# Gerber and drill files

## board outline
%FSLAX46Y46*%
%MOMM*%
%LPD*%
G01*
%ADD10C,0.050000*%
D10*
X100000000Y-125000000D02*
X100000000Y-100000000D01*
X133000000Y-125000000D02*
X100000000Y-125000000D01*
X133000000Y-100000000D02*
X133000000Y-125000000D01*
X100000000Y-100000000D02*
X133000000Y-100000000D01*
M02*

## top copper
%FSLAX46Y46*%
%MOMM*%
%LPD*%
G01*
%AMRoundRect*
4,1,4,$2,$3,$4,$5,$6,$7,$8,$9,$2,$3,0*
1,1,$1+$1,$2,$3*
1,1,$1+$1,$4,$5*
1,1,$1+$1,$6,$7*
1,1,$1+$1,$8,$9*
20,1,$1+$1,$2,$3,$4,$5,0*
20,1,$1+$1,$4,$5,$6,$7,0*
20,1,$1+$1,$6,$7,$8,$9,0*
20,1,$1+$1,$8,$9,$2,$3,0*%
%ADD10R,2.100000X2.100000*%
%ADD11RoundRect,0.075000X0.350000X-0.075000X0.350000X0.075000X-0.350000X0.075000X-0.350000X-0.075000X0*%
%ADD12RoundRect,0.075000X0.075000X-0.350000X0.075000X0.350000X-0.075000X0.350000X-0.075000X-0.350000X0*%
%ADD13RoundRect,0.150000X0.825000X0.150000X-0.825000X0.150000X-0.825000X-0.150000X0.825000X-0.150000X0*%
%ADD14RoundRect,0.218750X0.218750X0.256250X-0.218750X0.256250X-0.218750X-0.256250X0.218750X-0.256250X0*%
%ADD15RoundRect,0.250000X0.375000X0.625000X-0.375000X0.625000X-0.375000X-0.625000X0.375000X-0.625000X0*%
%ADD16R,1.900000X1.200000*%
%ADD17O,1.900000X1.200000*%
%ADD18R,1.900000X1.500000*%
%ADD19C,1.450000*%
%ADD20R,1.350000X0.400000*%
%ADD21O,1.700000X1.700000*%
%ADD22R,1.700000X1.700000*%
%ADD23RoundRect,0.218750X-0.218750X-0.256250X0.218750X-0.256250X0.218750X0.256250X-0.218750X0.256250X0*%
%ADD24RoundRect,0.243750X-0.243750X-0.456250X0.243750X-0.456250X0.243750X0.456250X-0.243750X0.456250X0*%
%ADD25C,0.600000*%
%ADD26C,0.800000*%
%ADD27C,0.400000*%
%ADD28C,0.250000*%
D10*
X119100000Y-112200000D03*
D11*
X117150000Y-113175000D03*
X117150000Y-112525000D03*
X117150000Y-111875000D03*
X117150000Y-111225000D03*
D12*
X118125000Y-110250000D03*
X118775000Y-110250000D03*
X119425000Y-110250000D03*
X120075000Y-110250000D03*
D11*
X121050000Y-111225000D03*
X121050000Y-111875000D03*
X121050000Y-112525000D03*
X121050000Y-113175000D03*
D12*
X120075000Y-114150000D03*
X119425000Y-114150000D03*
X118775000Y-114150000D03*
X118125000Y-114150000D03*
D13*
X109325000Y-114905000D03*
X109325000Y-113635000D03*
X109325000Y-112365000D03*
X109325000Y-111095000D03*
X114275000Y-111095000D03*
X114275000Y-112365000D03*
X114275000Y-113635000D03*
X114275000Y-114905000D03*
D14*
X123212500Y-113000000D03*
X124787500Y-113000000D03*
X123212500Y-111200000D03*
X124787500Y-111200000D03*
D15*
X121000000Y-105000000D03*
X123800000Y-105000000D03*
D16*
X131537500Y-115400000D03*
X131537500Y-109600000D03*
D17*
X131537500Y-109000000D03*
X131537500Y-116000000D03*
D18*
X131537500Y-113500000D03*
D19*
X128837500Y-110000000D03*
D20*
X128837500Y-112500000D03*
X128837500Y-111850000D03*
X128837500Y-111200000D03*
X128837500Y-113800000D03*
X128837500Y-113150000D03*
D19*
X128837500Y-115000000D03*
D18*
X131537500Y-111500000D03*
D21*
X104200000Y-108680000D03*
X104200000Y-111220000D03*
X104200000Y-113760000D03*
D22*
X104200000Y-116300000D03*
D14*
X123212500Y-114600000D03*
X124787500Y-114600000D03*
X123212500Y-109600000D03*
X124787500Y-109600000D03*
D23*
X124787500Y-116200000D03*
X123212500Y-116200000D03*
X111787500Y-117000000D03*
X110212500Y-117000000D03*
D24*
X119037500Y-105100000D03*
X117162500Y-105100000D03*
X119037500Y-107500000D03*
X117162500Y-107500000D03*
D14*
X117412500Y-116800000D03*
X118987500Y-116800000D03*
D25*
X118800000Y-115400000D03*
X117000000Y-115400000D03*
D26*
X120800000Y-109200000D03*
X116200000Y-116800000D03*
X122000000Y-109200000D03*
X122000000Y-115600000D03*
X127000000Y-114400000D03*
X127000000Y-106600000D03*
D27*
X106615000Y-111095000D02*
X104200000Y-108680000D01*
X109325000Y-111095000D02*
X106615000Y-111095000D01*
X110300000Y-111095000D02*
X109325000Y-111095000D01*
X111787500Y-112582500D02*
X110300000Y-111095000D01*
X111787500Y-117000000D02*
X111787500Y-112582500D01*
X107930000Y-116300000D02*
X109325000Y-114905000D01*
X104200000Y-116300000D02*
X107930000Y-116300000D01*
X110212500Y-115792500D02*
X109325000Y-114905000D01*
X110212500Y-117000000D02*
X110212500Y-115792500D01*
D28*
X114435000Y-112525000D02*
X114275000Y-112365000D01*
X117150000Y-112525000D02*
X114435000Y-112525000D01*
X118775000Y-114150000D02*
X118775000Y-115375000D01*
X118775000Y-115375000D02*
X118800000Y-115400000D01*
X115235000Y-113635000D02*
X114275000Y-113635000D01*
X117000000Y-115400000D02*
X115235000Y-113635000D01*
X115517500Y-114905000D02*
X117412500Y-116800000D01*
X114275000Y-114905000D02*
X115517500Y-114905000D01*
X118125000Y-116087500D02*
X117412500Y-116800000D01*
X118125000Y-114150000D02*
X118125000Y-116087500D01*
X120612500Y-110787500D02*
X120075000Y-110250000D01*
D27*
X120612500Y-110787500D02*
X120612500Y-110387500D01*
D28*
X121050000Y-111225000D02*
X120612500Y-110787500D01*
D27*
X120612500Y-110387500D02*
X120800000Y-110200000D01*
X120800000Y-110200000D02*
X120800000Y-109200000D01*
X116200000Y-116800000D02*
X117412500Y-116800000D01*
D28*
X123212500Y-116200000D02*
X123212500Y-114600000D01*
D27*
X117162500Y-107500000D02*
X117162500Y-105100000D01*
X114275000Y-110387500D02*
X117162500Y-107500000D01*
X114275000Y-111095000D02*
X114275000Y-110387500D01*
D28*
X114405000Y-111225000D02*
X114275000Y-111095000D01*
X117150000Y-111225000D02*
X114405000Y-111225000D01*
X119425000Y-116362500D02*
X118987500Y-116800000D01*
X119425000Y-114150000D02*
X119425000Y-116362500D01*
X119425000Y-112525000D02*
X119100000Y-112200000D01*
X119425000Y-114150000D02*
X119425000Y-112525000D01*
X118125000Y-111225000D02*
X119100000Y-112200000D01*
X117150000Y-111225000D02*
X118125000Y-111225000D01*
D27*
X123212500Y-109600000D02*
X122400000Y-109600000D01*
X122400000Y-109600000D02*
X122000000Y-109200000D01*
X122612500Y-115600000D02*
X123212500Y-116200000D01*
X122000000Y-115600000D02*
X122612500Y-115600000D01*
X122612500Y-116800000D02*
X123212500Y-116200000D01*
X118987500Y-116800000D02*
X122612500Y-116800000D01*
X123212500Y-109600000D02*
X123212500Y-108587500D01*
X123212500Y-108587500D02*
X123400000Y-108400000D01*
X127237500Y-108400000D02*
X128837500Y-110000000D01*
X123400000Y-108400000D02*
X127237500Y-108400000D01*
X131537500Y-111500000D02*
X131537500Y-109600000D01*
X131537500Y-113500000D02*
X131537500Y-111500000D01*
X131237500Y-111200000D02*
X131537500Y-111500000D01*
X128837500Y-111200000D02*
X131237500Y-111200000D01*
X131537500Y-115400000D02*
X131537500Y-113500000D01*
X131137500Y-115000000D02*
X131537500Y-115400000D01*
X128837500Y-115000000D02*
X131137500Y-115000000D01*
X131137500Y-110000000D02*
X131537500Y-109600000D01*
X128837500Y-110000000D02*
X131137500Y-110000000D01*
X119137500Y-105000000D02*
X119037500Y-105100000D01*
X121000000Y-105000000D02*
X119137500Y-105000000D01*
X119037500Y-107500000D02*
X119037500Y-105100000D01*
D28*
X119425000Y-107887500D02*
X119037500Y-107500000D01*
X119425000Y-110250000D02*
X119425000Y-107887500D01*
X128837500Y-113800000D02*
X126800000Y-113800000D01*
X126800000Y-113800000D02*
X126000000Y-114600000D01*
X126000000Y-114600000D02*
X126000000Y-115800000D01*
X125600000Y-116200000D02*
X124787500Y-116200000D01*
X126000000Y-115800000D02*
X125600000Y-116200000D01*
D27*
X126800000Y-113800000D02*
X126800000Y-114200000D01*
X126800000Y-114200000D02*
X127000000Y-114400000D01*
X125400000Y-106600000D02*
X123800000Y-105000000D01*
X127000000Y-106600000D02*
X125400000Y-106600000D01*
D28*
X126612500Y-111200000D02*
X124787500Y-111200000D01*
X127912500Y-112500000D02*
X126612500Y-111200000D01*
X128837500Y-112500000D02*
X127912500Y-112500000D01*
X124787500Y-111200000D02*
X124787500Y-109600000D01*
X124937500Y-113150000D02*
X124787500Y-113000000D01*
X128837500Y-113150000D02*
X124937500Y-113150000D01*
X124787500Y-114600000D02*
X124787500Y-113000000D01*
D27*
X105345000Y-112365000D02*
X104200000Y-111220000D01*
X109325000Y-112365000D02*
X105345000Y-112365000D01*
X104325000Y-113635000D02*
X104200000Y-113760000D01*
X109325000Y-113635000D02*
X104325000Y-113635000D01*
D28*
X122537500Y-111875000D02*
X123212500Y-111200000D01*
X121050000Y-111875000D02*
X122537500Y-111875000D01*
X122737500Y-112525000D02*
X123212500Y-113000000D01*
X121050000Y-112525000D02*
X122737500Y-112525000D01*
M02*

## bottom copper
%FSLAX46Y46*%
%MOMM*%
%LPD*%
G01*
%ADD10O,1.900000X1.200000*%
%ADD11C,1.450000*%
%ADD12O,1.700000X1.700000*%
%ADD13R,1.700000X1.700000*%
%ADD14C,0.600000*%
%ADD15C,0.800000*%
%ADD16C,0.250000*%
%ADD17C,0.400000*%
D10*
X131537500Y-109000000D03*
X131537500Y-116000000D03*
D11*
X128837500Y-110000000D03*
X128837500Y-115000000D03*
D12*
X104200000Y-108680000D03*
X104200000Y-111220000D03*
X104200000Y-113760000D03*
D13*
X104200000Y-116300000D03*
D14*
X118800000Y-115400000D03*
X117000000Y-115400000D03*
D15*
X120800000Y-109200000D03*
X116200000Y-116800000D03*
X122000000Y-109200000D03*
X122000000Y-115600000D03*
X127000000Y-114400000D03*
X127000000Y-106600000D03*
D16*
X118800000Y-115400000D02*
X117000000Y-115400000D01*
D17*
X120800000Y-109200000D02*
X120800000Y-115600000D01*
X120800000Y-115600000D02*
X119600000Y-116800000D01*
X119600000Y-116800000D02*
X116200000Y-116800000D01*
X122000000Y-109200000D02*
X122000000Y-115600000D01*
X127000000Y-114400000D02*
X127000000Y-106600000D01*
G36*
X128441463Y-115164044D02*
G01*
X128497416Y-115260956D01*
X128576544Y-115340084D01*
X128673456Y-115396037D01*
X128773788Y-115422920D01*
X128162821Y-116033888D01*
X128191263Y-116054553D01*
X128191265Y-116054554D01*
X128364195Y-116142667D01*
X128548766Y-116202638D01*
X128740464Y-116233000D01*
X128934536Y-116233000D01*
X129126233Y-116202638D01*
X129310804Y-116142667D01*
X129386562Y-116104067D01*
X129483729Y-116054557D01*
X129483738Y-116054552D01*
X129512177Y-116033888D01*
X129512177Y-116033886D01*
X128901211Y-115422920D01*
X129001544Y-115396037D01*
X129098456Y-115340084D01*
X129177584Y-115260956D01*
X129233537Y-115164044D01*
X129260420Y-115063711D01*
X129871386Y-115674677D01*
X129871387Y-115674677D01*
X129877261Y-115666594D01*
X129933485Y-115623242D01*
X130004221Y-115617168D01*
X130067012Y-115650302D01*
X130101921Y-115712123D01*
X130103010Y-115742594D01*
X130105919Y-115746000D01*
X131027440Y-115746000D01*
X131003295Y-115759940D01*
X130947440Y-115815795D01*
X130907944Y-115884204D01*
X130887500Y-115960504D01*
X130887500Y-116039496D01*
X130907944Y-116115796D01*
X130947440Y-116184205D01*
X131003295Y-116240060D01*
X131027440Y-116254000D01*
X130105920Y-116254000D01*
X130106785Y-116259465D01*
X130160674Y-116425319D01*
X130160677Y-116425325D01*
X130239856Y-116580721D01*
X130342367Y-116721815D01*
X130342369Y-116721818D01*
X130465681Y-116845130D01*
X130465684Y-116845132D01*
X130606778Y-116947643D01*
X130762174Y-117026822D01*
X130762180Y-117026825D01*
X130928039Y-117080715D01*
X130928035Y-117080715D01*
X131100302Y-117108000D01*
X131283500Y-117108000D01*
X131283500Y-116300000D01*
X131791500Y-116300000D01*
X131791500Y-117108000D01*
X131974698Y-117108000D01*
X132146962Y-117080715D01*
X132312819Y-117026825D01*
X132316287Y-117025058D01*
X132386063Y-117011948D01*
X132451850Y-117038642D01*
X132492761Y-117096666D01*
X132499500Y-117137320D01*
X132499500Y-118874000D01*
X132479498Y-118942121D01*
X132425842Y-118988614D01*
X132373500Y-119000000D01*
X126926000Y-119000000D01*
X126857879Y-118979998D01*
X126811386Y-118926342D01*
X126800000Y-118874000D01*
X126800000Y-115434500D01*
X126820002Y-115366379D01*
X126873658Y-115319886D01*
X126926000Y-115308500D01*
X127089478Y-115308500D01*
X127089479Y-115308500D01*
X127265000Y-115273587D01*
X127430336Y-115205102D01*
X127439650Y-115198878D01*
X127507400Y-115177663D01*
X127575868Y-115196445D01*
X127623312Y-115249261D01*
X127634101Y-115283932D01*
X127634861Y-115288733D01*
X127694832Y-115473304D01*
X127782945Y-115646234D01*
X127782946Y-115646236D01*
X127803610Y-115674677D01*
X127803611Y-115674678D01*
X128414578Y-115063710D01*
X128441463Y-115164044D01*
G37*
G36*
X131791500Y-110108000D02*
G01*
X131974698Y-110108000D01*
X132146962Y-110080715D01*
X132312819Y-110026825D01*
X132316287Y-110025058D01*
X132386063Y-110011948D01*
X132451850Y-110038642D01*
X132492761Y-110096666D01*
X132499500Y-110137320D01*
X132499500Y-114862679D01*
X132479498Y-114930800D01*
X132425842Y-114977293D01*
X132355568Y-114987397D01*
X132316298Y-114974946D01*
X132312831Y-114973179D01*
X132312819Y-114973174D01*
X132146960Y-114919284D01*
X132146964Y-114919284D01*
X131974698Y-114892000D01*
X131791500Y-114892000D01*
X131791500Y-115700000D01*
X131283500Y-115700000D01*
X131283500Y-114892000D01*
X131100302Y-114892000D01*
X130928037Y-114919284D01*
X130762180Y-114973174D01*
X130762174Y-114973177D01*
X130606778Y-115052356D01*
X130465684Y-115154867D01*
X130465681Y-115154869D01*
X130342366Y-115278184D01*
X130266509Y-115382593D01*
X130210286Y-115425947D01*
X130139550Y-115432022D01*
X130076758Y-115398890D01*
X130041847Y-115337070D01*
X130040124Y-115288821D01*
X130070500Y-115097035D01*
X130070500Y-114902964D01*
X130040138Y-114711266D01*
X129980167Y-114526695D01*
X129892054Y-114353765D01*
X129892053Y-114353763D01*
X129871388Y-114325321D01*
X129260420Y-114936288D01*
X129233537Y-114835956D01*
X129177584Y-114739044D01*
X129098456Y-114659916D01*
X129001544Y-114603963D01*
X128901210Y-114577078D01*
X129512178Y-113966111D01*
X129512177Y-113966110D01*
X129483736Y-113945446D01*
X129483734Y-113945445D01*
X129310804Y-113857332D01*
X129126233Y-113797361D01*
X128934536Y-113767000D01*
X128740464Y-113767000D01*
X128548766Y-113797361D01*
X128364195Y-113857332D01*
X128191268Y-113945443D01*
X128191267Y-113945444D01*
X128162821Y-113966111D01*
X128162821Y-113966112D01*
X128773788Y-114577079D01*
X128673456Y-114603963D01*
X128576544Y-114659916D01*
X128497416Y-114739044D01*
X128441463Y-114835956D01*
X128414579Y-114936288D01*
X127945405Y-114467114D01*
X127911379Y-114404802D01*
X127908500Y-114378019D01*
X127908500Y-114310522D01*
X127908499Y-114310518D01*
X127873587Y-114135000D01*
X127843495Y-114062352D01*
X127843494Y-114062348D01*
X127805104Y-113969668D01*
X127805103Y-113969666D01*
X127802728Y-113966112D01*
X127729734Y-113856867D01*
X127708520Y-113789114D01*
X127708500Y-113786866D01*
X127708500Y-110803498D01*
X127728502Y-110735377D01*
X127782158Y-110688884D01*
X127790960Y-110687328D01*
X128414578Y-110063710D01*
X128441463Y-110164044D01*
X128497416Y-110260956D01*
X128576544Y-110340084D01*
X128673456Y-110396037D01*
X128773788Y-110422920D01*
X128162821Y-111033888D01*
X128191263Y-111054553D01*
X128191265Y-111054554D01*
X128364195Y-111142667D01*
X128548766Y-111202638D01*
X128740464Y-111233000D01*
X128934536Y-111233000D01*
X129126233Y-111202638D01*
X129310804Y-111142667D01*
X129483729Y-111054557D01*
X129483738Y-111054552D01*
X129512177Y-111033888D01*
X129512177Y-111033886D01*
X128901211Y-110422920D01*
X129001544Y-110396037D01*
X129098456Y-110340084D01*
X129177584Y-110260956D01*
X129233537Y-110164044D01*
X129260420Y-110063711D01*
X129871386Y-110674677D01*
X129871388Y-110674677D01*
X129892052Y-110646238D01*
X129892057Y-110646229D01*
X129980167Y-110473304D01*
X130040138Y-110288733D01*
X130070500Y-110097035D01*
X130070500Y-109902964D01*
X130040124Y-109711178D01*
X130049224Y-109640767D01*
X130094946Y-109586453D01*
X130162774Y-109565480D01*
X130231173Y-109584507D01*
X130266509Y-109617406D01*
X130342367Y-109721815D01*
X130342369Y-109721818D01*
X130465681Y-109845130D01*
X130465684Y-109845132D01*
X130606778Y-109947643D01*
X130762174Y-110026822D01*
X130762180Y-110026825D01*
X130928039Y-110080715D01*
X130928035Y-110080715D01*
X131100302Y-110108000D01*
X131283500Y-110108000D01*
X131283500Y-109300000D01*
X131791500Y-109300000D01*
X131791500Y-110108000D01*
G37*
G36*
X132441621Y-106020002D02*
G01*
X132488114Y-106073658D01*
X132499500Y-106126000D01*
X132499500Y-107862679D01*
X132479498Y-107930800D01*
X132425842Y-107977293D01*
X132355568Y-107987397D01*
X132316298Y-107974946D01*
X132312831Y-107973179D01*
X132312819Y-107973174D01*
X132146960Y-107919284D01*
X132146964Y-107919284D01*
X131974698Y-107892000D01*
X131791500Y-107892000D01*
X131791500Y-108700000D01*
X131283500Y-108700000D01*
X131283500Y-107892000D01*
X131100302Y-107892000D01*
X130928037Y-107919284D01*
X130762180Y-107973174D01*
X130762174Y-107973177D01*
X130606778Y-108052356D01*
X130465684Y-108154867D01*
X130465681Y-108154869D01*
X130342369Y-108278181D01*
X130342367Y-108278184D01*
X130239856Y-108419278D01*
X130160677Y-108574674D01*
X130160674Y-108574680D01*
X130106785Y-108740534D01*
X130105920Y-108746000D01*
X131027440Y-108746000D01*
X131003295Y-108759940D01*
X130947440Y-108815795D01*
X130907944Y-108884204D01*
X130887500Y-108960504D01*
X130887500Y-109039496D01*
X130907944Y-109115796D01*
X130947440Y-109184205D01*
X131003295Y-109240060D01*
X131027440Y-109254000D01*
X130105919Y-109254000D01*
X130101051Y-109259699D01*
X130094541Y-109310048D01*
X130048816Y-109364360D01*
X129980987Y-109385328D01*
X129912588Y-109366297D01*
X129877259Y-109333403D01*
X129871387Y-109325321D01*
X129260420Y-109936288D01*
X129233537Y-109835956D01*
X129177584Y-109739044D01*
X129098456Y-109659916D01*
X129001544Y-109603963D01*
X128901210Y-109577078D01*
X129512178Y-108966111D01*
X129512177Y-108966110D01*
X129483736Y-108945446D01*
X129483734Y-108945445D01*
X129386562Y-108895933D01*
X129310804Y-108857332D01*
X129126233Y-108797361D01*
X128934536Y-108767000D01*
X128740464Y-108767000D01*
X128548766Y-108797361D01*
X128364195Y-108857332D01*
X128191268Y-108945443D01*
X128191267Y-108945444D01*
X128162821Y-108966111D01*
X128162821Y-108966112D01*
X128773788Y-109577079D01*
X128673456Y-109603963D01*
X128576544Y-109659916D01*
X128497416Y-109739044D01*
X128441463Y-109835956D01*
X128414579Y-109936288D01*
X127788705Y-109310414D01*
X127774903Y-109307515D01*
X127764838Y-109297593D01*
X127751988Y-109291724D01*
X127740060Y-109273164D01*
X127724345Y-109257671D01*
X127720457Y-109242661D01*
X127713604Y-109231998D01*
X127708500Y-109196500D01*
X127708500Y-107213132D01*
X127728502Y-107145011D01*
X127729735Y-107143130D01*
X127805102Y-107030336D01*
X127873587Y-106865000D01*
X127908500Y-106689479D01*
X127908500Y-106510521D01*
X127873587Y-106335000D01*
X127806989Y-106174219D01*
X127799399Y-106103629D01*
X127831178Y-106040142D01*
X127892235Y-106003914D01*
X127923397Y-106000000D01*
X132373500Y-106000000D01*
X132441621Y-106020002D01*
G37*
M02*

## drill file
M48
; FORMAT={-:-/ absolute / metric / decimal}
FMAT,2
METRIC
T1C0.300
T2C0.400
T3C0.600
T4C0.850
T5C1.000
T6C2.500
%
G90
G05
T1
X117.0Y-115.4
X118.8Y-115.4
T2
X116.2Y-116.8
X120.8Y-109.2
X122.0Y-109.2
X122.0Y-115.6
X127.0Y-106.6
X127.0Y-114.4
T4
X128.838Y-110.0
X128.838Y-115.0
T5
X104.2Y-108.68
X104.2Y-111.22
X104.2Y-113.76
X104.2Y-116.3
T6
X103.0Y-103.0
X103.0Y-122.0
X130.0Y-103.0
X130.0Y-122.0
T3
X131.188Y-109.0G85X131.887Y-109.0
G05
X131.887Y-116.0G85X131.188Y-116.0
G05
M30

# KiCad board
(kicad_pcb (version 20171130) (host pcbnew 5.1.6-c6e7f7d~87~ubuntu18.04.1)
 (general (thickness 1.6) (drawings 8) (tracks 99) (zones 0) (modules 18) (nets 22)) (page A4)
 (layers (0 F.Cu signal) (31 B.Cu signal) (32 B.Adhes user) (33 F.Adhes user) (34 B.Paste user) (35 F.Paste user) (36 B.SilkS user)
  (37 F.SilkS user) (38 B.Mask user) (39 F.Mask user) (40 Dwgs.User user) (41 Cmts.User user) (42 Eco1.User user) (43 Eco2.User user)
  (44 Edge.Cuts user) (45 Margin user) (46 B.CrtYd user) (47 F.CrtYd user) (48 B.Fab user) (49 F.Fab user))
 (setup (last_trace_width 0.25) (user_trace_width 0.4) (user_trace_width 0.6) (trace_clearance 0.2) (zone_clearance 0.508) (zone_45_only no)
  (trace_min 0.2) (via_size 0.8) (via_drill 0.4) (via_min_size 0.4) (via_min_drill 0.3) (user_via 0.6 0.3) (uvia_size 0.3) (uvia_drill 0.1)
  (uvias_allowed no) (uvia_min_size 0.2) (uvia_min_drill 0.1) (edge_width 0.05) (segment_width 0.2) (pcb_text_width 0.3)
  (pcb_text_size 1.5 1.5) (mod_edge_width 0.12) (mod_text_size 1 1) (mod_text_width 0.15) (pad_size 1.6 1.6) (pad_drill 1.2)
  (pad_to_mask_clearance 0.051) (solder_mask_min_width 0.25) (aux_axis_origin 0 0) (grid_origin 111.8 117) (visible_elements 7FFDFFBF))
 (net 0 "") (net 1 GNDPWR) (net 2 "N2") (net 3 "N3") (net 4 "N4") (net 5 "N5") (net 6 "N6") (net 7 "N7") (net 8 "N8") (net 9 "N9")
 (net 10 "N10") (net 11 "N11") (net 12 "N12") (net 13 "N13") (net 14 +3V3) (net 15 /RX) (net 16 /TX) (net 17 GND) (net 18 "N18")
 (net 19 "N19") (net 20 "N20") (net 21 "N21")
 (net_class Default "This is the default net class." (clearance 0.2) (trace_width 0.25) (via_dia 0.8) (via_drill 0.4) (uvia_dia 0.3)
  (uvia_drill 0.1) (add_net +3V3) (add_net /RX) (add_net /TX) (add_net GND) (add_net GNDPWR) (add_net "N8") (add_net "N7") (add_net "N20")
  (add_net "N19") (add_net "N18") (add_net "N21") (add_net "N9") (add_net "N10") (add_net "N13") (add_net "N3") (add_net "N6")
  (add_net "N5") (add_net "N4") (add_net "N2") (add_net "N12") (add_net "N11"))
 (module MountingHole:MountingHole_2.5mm (layer F.Cu) (at 130 122)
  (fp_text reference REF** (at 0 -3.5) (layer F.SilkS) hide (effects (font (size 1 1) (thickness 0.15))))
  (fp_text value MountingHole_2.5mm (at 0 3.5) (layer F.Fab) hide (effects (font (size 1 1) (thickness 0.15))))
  (pad 1 np_thru_hole circle (at 0 0) (size 2.5 2.5) (drill 2.5) (layers *.Cu *.Mask)))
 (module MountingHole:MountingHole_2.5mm (layer F.Cu) (at 130 103)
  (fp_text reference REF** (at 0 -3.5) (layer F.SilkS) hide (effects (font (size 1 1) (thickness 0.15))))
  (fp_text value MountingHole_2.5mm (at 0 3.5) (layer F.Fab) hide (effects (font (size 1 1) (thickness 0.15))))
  (pad 1 np_thru_hole circle (at 0 0) (size 2.5 2.5) (drill 2.5) (layers *.Cu *.Mask)))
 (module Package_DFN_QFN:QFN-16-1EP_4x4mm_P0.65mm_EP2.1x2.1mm (layer F.Cu) (at 119.1 112.2 90)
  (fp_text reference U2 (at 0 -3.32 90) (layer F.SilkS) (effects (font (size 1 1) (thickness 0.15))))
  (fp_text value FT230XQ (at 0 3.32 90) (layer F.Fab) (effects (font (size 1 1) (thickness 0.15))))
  (pad "" smd roundrect (at 0.525 0.525 90) (size 0.85 0.85) (layers F.Paste) (roundrect_rratio 0.25))
  (pad "" smd roundrect (at 0.525 -0.525 90) (size 0.85 0.85) (layers F.Paste) (roundrect_rratio 0.25))
  (pad "" smd roundrect (at -0.525 0.525 90) (size 0.85 0.85) (layers F.Paste) (roundrect_rratio 0.25))
  (pad "" smd roundrect (at -0.525 -0.525 90) (size 0.85 0.85) (layers F.Paste) (roundrect_rratio 0.25))
  (pad 17 smd rect (at 0 0 90) (size 2.1 2.1) (layers F.Cu F.Mask) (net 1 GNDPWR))
  (pad 16 smd roundrect (at -0.975 -1.95 90) (size 0.3 0.85) (layers F.Cu F.Paste F.Mask) (roundrect_rratio 0.25) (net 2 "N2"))
  (pad 15 smd roundrect (at -0.325 -1.95 90) (size 0.3 0.85) (layers F.Cu F.Paste F.Mask) (roundrect_rratio 0.25) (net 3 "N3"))
  (pad 14 smd roundrect (at 0.325 -1.95 90) (size 0.3 0.85) (layers F.Cu F.Paste F.Mask) (roundrect_rratio 0.25) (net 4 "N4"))
  (pad 13 smd roundrect (at 0.975 -1.95 90) (size 0.3 0.85) (layers F.Cu F.Paste F.Mask) (roundrect_rratio 0.25) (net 1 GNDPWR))
  (pad 12 smd roundrect (at 1.95 -0.975 90) (size 0.85 0.3) (layers F.Cu F.Paste F.Mask) (roundrect_rratio 0.25) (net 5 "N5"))
  (pad 11 smd roundrect (at 1.95 -0.325 90) (size 0.85 0.3) (layers F.Cu F.Paste F.Mask) (roundrect_rratio 0.25) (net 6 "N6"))
  (pad 10 smd roundrect (at 1.95 0.325 90) (size 0.85 0.3) (layers F.Cu F.Paste F.Mask) (roundrect_rratio 0.25) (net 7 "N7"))
  (pad 9 smd roundrect (at 1.95 0.975 90) (size 0.85 0.3) (layers F.Cu F.Paste F.Mask) (roundrect_rratio 0.25) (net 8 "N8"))
  (pad 8 smd roundrect (at 0.975 1.95 90) (size 0.3 0.85) (layers F.Cu F.Paste F.Mask) (roundrect_rratio 0.25) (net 8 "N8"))
  (pad 7 smd roundrect (at 0.325 1.95 90) (size 0.3 0.85) (layers F.Cu F.Paste F.Mask) (roundrect_rratio 0.25) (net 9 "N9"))
  (pad 6 smd roundrect (at -0.325 1.95 90) (size 0.3 0.85) (layers F.Cu F.Paste F.Mask) (roundrect_rratio 0.25) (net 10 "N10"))
  (pad 5 smd roundrect (at -0.975 1.95 90) (size 0.3 0.85) (layers F.Cu F.Paste F.Mask) (roundrect_rratio 0.25) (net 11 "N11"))
  (pad 4 smd roundrect (at -1.95 0.975 90) (size 0.85 0.3) (layers F.Cu F.Paste F.Mask) (roundrect_rratio 0.25) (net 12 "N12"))
  (pad 3 smd roundrect (at -1.95 0.325 90) (size 0.85 0.3) (layers F.Cu F.Paste F.Mask) (roundrect_rratio 0.25) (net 1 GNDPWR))
  (pad 2 smd roundrect (at -1.95 -0.325 90) (size 0.85 0.3) (layers F.Cu F.Paste F.Mask) (roundrect_rratio 0.25) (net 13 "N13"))
  (pad 1 smd roundrect (at -1.95 -0.975 90) (size 0.85 0.3) (layers F.Cu F.Paste F.Mask) (roundrect_rratio 0.25) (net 8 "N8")))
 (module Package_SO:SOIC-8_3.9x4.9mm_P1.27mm (layer F.Cu) (at 111.8 113 180)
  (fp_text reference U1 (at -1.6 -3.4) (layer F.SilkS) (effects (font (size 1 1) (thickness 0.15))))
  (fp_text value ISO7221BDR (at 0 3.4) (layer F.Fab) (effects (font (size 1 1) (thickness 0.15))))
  (pad 8 smd roundrect (at 2.475 -1.905 180) (size 1.95 0.6) (layers F.Cu F.Paste F.Mask) (roundrect_rratio 0.25) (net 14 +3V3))
  (pad 7 smd roundrect (at 2.475 -0.635 180) (size 1.95 0.6) (layers F.Cu F.Paste F.Mask) (roundrect_rratio 0.25) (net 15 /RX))
  (pad 6 smd roundrect (at 2.475 0.635 180) (size 1.95 0.6) (layers F.Cu F.Paste F.Mask) (roundrect_rratio 0.25) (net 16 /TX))
  (pad 5 smd roundrect (at 2.475 1.905 180) (size 1.95 0.6) (layers F.Cu F.Paste F.Mask) (roundrect_rratio 0.25) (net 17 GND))
  (pad 4 smd roundrect (at -2.475 1.905 180) (size 1.95 0.6) (layers F.Cu F.Paste F.Mask) (roundrect_rratio 0.25) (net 1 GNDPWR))
  (pad 3 smd roundrect (at -2.475 0.635 180) (size 1.95 0.6) (layers F.Cu F.Paste F.Mask) (roundrect_rratio 0.25) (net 3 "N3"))
  (pad 2 smd roundrect (at -2.475 -0.635 180) (size 1.95 0.6) (layers F.Cu F.Paste F.Mask) (roundrect_rratio 0.25) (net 13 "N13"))
  (pad 1 smd roundrect (at -2.475 -1.905 180) (size 1.95 0.6) (layers F.Cu F.Paste F.Mask) (roundrect_rratio 0.25) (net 8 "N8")))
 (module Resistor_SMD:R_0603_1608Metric (layer F.Cu) (at 124 113 180)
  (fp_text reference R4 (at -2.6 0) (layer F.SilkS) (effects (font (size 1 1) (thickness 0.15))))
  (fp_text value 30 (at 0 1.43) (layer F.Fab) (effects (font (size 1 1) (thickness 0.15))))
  (pad 2 smd roundrect (at 0.7875 0 180) (size 0.875 0.95) (layers F.Cu F.Paste F.Mask) (roundrect_rratio 0.25) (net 10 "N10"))
  (pad 1 smd roundrect (at -0.7875 0 180) (size 0.875 0.95) (layers F.Cu F.Paste F.Mask) (roundrect_rratio 0.25) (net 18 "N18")))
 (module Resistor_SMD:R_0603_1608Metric (layer F.Cu) (at 124 111.2 180)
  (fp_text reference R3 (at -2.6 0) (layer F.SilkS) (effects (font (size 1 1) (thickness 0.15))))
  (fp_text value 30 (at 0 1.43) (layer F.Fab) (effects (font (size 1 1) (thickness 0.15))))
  (pad 2 smd roundrect (at 0.7875 0 180) (size 0.875 0.95) (layers F.Cu F.Paste F.Mask) (roundrect_rratio 0.25) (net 9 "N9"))
  (pad 1 smd roundrect (at -0.7875 0 180) (size 0.875 0.95) (layers F.Cu F.Paste F.Mask) (roundrect_rratio 0.25) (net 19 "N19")))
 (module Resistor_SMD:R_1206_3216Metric (layer F.Cu) (at 122.4 105 180)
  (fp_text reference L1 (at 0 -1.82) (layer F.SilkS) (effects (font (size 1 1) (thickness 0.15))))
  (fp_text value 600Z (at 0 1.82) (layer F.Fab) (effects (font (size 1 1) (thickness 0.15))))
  (pad 2 smd roundrect (at 1.4 0 180) (size 1.25 1.75) (layers F.Cu F.Paste F.Mask) (roundrect_rratio 0.2) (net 7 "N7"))
  (pad 1 smd roundrect (at -1.4 0 180) (size 1.25 1.75) (layers F.Cu F.Paste F.Mask) (roundrect_rratio 0.2) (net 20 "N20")))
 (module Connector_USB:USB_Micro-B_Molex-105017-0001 (layer F.Cu) (at 130.3 112.5 90)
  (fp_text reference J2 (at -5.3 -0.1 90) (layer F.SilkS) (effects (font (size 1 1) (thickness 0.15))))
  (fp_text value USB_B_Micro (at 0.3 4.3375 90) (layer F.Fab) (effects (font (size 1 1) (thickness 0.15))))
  (pad 6 smd rect (at -2.9 1.2375 90) (size 1.2 1.9) (layers F.Cu F.Mask) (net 1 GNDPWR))
  (pad 6 smd rect (at 2.9 1.2375 90) (size 1.2 1.9) (layers F.Cu F.Mask) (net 1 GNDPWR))
  (pad 6 thru_hole oval (at 3.5 1.2375 90) (size 1.2 1.9) (drill oval 0.6 1.3) (layers *.Cu *.Mask) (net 1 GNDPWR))
  (pad 6 thru_hole oval (at -3.5 1.2375 270) (size 1.2 1.9) (drill oval 0.6 1.3) (layers *.Cu *.Mask) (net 1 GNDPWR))
  (pad 6 smd rect (at -1 1.2375 90) (size 1.5 1.9) (layers F.Cu F.Paste F.Mask) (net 1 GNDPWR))
  (pad 6 thru_hole circle (at 2.5 -1.4625 90) (size 1.45 1.45) (drill 0.85) (layers *.Cu *.Mask) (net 1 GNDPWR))
  (pad 3 smd rect (at 0 -1.4625 90) (size 0.4 1.35) (layers F.Cu F.Paste F.Mask) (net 19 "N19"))
  (pad 4 smd rect (at 0.65 -1.4625 90) (size 0.4 1.35) (layers F.Cu F.Paste F.Mask) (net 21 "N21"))
  (pad 5 smd rect (at 1.3 -1.4625 90) (size 0.4 1.35) (layers F.Cu F.Paste F.Mask) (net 1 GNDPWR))
  (pad 1 smd rect (at -1.3 -1.4625 90) (size 0.4 1.35) (layers F.Cu F.Paste F.Mask) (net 20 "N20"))
  (pad 2 smd rect (at -0.65 -1.4625 90) (size 0.4 1.35) (layers F.Cu F.Paste F.Mask) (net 18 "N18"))
  (pad 6 thru_hole circle (at -2.5 -1.4625 90) (size 1.45 1.45) (drill 0.85) (layers *.Cu *.Mask) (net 1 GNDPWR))
  (pad 6 smd rect (at 1 1.2375 90) (size 1.5 1.9) (layers F.Cu F.Paste F.Mask) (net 1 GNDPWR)))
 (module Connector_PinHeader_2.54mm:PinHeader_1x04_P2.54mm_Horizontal (layer F.Cu) (at 104.2 116.3 180)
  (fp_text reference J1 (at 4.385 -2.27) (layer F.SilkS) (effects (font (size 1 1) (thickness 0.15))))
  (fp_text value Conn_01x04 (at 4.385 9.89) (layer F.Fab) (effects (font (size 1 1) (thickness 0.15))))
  (pad 4 thru_hole oval (at 0 7.62 180) (size 1.7 1.7) (drill 1) (layers *.Cu *.Mask) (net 17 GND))
  (pad 3 thru_hole oval (at 0 5.08 180) (size 1.7 1.7) (drill 1) (layers *.Cu *.Mask) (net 16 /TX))
  (pad 2 thru_hole oval (at 0 2.54 180) (size 1.7 1.7) (drill 1) (layers *.Cu *.Mask) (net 15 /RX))
  (pad 1 thru_hole rect (at 0 0 180) (size 1.7 1.7) (drill 1) (layers *.Cu *.Mask) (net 14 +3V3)))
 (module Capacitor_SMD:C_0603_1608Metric (layer F.Cu) (at 124 114.6 180)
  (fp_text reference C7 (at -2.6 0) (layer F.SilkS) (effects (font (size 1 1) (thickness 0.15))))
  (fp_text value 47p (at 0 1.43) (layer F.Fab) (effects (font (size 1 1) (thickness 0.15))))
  (pad 2 smd roundrect (at 0.7875 0 180) (size 0.875 0.95) (layers F.Cu F.Paste F.Mask) (roundrect_rratio 0.25) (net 1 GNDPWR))
  (pad 1 smd roundrect (at -0.7875 0 180) (size 0.875 0.95) (layers F.Cu F.Paste F.Mask) (roundrect_rratio 0.25) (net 18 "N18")))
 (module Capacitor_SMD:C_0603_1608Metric (layer F.Cu) (at 124 109.6 180)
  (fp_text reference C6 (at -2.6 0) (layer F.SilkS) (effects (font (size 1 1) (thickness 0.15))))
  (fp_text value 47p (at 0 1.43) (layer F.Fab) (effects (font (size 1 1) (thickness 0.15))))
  (pad 2 smd roundrect (at 0.7875 0 180) (size 0.875 0.95) (layers F.Cu F.Paste F.Mask) (roundrect_rratio 0.25) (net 1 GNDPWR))
  (pad 1 smd roundrect (at -0.7875 0 180) (size 0.875 0.95) (layers F.Cu F.Paste F.Mask) (roundrect_rratio 0.25) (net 19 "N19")))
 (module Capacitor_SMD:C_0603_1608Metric (layer F.Cu) (at 124 116.2)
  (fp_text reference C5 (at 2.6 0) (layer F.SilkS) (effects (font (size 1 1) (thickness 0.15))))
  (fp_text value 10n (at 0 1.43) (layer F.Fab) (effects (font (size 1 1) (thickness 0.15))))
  (pad 2 smd roundrect (at 0.7875 0) (size 0.875 0.95) (layers F.Cu F.Paste F.Mask) (roundrect_rratio 0.25) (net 20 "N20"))
  (pad 1 smd roundrect (at -0.7875 0) (size 0.875 0.95) (layers F.Cu F.Paste F.Mask) (roundrect_rratio 0.25) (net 1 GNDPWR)))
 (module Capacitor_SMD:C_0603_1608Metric (layer F.Cu) (at 111 117)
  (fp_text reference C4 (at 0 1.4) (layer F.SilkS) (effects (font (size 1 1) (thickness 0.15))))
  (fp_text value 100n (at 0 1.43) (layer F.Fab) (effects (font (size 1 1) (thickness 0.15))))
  (pad 2 smd roundrect (at 0.7875 0) (size 0.875 0.95) (layers F.Cu F.Paste F.Mask) (roundrect_rratio 0.25) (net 17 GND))
  (pad 1 smd roundrect (at -0.7875 0) (size 0.875 0.95) (layers F.Cu F.Paste F.Mask) (roundrect_rratio 0.25) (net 14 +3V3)))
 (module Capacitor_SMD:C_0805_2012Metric (layer F.Cu) (at 118.1 105.1)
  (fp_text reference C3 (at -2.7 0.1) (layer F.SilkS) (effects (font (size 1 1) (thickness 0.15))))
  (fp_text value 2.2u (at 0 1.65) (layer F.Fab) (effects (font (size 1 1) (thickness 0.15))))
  (pad 2 smd roundrect (at 0.9375 0) (size 0.975 1.4) (layers F.Cu F.Paste F.Mask) (roundrect_rratio 0.25) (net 7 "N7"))
  (pad 1 smd roundrect (at -0.9375 0) (size 0.975 1.4) (layers F.Cu F.Paste F.Mask) (roundrect_rratio 0.25) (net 1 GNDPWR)))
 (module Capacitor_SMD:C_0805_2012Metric (layer F.Cu) (at 118.1 107.5)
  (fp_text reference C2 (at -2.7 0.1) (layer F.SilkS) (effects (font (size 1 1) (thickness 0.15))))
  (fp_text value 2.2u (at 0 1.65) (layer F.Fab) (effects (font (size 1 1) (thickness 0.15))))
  (pad 2 smd roundrect (at 0.9375 0) (size 0.975 1.4) (layers F.Cu F.Paste F.Mask) (roundrect_rratio 0.25) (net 7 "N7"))
  (pad 1 smd roundrect (at -0.9375 0) (size 0.975 1.4) (layers F.Cu F.Paste F.Mask) (roundrect_rratio 0.25) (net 1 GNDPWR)))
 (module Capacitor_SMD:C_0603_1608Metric (layer F.Cu) (at 118.2 116.8 180)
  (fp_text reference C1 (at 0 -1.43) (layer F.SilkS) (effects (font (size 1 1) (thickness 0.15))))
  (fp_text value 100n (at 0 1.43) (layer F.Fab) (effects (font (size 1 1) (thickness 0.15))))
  (pad 2 smd roundrect (at 0.7875 0 180) (size 0.875 0.95) (layers F.Cu F.Paste F.Mask) (roundrect_rratio 0.25) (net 8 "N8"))
  (pad 1 smd roundrect (at -0.7875 0 180) (size 0.875 0.95) (layers F.Cu F.Paste F.Mask) (roundrect_rratio 0.25) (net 1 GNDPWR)))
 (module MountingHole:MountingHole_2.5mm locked (layer F.Cu) (at 103 122)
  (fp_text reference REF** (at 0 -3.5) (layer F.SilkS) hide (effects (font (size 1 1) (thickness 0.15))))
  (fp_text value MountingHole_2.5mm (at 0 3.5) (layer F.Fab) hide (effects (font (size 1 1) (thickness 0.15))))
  (pad 1 np_thru_hole circle (at 0 0) (size 2.5 2.5) (drill 2.5) (layers *.Cu *.Mask)))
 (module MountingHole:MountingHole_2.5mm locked (layer F.Cu) (at 103 103)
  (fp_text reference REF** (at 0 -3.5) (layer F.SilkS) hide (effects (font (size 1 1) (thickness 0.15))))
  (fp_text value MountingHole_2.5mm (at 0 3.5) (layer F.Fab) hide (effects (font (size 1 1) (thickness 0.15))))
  (pad 1 np_thru_hole circle (at 0 0) (size 2.5 2.5) (drill 2.5) (layers *.Cu *.Mask)))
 (gr_line (start 100 125) (end 100 100) (layer Edge.Cuts) (width 0.05))
 (gr_line (start 133 125) (end 100 125) (layer Edge.Cuts) (width 0.05))
 (gr_line (start 133 100) (end 133 125) (layer Edge.Cuts) (width 0.05))
 (gr_line (start 100 100) (end 133 100) (layer Edge.Cuts) (width 0.05))
 (segment (start 106.615 111.095) (end 104.2 108.68) (width 0.4) (layer F.Cu) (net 17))
 (segment (start 109.325 111.095) (end 106.615 111.095) (width 0.4) (layer F.Cu) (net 17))
 (segment (start 110.3 111.095) (end 109.325 111.095) (width 0.4) (layer F.Cu) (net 17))
 (segment (start 111.7875 112.5825) (end 110.3 111.095) (width 0.4) (layer F.Cu) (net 17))
 (segment (start 111.7875 117) (end 111.7875 112.5825) (width 0.4) (layer F.Cu) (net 17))
 (segment (start 107.93 116.3) (end 109.325 114.905) (width 0.4) (layer F.Cu) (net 14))
 (segment (start 104.2 116.3) (end 107.93 116.3) (width 0.4) (layer F.Cu) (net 14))
 (segment (start 110.2125 115.7925) (end 109.325 114.905) (width 0.4) (layer F.Cu) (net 14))
 (segment (start 110.2125 117) (end 110.2125 115.7925) (width 0.4) (layer F.Cu) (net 14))
 (segment (start 114.435 112.525) (end 114.275 112.365) (width 0.25) (layer F.Cu) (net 3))
 (segment (start 117.15 112.525) (end 114.435 112.525) (width 0.25) (layer F.Cu) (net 3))
 (via (at 118.8 115.4) (size 0.6) (drill 0.3) (layers F.Cu B.Cu) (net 13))
 (segment (start 118.775 114.15) (end 118.775 115.375) (width 0.25) (layer F.Cu) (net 13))
 (segment (start 118.775 115.375) (end 118.8 115.4) (width 0.25) (layer F.Cu) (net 13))
 (via (at 117 115.4) (size 0.6) (drill 0.3) (layers F.Cu B.Cu) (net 13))
 (segment (start 118.8 115.4) (end 117 115.4) (width 0.25) (layer B.Cu) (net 13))
 (segment (start 115.235 113.635) (end 114.275 113.635) (width 0.25) (layer F.Cu) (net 13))
 (segment (start 117 115.4) (end 115.235 113.635) (width 0.25) (layer F.Cu) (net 13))
 (segment (start 115.5175 114.905) (end 117.4125 116.8) (width 0.25) (layer F.Cu) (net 8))
 (segment (start 114.275 114.905) (end 115.5175 114.905) (width 0.25) (layer F.Cu) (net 8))
 (segment (start 118.125 116.0875) (end 117.4125 116.8) (width 0.25) (layer F.Cu) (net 8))
 (segment (start 118.125 114.15) (end 118.125 116.0875) (width 0.25) (layer F.Cu) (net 8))
 (segment (start 120.6125 110.7875) (end 120.075 110.25) (width 0.25) (layer F.Cu) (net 8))
 (segment (start 120.6125 110.7875) (end 120.6125 110.3875) (width 0.4) (layer F.Cu) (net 8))
 (segment (start 121.05 111.225) (end 120.6125 110.7875) (width 0.25) (layer F.Cu) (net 8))
 (via (at 120.8 109.2) (size 0.8) (drill 0.4) (layers F.Cu B.Cu) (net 8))
 (segment (start 120.6125 110.3875) (end 120.8 110.2) (width 0.4) (layer F.Cu) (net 8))
 (segment (start 120.8 110.2) (end 120.8 109.2) (width 0.4) (layer F.Cu) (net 8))
 (segment (start 120.8 109.2) (end 120.8 115.6) (width 0.4) (layer B.Cu) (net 8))
 (via (at 116.2 116.8) (size 0.8) (drill 0.4) (layers F.Cu B.Cu) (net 8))
 (segment (start 120.8 115.6) (end 119.6 116.8) (width 0.4) (layer B.Cu) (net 8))
 (segment (start 119.6 116.8) (end 116.2 116.8) (width 0.4) (layer B.Cu) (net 8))
 (segment (start 116.2 116.8) (end 117.4125 116.8) (width 0.4) (layer F.Cu) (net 8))
 (segment (start 123.2125 116.2) (end 123.2125 114.6) (width 0.25) (layer F.Cu) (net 1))
 (segment (start 117.1625 107.5) (end 117.1625 105.1) (width 0.4) (layer F.Cu) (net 1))
 (segment (start 114.275 110.3875) (end 117.1625 107.5) (width 0.4) (layer F.Cu) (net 1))
 (segment (start 114.275 111.095) (end 114.275 110.3875) (width 0.4) (layer F.Cu) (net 1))
 (segment (start 114.405 111.225) (end 114.275 111.095) (width 0.25) (layer F.Cu) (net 1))
 (segment (start 117.15 111.225) (end 114.405 111.225) (width 0.25) (layer F.Cu) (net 1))
 (segment (start 119.425 116.3625) (end 118.9875 116.8) (width 0.25) (layer F.Cu) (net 1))
 (segment (start 119.425 114.15) (end 119.425 116.3625) (width 0.25) (layer F.Cu) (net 1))
 (segment (start 119.425 112.525) (end 119.1 112.2) (width 0.25) (layer F.Cu) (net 1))
 (segment (start 119.425 114.15) (end 119.425 112.525) (width 0.25) (layer F.Cu) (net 1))
 (segment (start 118.125 111.225) (end 119.1 112.2) (width 0.25) (layer F.Cu) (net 1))
 (segment (start 117.15 111.225) (end 118.125 111.225) (width 0.25) (layer F.Cu) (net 1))
 (segment (start 123.2125 109.6) (end 122.4 109.6) (width 0.4) (layer F.Cu) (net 1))
 (via (at 122 109.2) (size 0.8) (drill 0.4) (layers F.Cu B.Cu) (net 1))
 (segment (start 122.4 109.6) (end 122 109.2) (width 0.4) (layer F.Cu) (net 1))
 (via (at 122 115.6) (size 0.8) (drill 0.4) (layers F.Cu B.Cu) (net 1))
 (segment (start 122 109.2) (end 122 115.6) (width 0.4) (layer B.Cu) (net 1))
 (segment (start 122.6125 115.6) (end 123.2125 116.2) (width 0.4) (layer F.Cu) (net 1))
 (segment (start 122 115.6) (end 122.6125 115.6) (width 0.4) (layer F.Cu) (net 1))
 (segment (start 122.6125 116.8) (end 123.2125 116.2) (width 0.4) (layer F.Cu) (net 1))
 (segment (start 118.9875 116.8) (end 122.6125 116.8) (width 0.4) (layer F.Cu) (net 1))
 (segment (start 123.2125 109.6) (end 123.2125 108.5875) (width 0.4) (layer F.Cu) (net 1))
 (segment (start 123.2125 108.5875) (end 123.4 108.4) (width 0.4) (layer F.Cu) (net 1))
 (segment (start 127.2375 108.4) (end 128.8375 110) (width 0.4) (layer F.Cu) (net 1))
 (segment (start 123.4 108.4) (end 127.2375 108.4) (width 0.4) (layer F.Cu) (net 1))
 (segment (start 131.5375 111.5) (end 131.5375 109.6) (width 0.4) (layer F.Cu) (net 1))
 (segment (start 131.5375 113.5) (end 131.5375 111.5) (width 0.4) (layer F.Cu) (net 1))
 (segment (start 131.2375 111.2) (end 131.5375 111.5) (width 0.4) (layer F.Cu) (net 1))
 (segment (start 128.8375 111.2) (end 131.2375 111.2) (width 0.4) (layer F.Cu) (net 1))
 (segment (start 131.5375 115.4) (end 131.5375 113.5) (width 0.4) (layer F.Cu) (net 1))
 (segment (start 131.1375 115) (end 131.5375 115.4) (width 0.4) (layer F.Cu) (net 1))
 (segment (start 128.8375 115) (end 131.1375 115) (width 0.4) (layer F.Cu) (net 1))
 (segment (start 131.1375 110) (end 131.5375 109.6) (width 0.4) (layer F.Cu) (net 1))
 (segment (start 128.8375 110) (end 131.1375 110) (width 0.4) (layer F.Cu) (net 1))
 (segment (start 119.1375 105) (end 119.0375 105.1) (width 0.4) (layer F.Cu) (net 7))
 (segment (start 121 105) (end 119.1375 105) (width 0.4) (layer F.Cu) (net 7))
 (segment (start 119.0375 107.5) (end 119.0375 105.1) (width 0.4) (layer F.Cu) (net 7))
 (segment (start 119.425 107.8875) (end 119.0375 107.5) (width 0.25) (layer F.Cu) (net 7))
 (segment (start 119.425 110.25) (end 119.425 107.8875) (width 0.25) (layer F.Cu) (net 7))
 (segment (start 128.8375 113.8) (end 126.8 113.8) (width 0.25) (layer F.Cu) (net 20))
 (segment (start 126.8 113.8) (end 126 114.6) (width 0.25) (layer F.Cu) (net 20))
 (segment (start 126 114.6) (end 126 115.8) (width 0.25) (layer F.Cu) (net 20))
 (segment (start 125.6 116.2) (end 124.7875 116.2) (width 0.25) (layer F.Cu) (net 20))
 (segment (start 126 115.8) (end 125.6 116.2) (width 0.25) (layer F.Cu) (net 20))
 (via (at 127 114.4) (size 0.8) (drill 0.4) (layers F.Cu B.Cu) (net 20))
 (segment (start 126.8 113.8) (end 126.8 114.2) (width 0.4) (layer F.Cu) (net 20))
 (segment (start 126.8 114.2) (end 127 114.4) (width 0.4) (layer F.Cu) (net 20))
 (via (at 127 106.6) (size 0.8) (drill 0.4) (layers F.Cu B.Cu) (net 20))
 (segment (start 127 114.4) (end 127 106.6) (width 0.4) (layer B.Cu) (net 20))
 (segment (start 125.4 106.6) (end 123.8 105) (width 0.4) (layer F.Cu) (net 20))
 (segment (start 127 106.6) (end 125.4 106.6) (width 0.4) (layer F.Cu) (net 20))
 (segment (start 126.6125 111.2) (end 124.7875 111.2) (width 0.25) (layer F.Cu) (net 19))
 (segment (start 127.9125 112.5) (end 126.6125 111.2) (width 0.25) (layer F.Cu) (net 19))
 (segment (start 128.8375 112.5) (end 127.9125 112.5) (width 0.25) (layer F.Cu) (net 19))
 (segment (start 124.7875 111.2) (end 124.7875 109.6) (width 0.25) (layer F.Cu) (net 19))
 (segment (start 124.9375 113.15) (end 124.7875 113) (width 0.25) (layer F.Cu) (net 18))
 (segment (start 128.8375 113.15) (end 124.9375 113.15) (width 0.25) (layer F.Cu) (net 18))
 (segment (start 124.7875 114.6) (end 124.7875 113) (width 0.25) (layer F.Cu) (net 18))
 (segment (start 105.345 112.365) (end 104.2 111.22) (width 0.4) (layer F.Cu) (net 16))
 (segment (start 109.325 112.365) (end 105.345 112.365) (width 0.4) (layer F.Cu) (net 16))
 (segment (start 104.325 113.635) (end 104.2 113.76) (width 0.4) (layer F.Cu) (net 15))
 (segment (start 109.325 113.635) (end 104.325 113.635) (width 0.4) (layer F.Cu) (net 15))
 (segment (start 122.5375 111.875) (end 123.2125 111.2) (width 0.25) (layer F.Cu) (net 9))
 (segment (start 121.05 111.875) (end 122.5375 111.875) (width 0.25) (layer F.Cu) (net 9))
 (segment (start 122.7375 112.525) (end 123.2125 113) (width 0.25) (layer F.Cu) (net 10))
 (segment (start 121.05 112.525) (end 122.7375 112.525) (width 0.25) (layer F.Cu) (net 10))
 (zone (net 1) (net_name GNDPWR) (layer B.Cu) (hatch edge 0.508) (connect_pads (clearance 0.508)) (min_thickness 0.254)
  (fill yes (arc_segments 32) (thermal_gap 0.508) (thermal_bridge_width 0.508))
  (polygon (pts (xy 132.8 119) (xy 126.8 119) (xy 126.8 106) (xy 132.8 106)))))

